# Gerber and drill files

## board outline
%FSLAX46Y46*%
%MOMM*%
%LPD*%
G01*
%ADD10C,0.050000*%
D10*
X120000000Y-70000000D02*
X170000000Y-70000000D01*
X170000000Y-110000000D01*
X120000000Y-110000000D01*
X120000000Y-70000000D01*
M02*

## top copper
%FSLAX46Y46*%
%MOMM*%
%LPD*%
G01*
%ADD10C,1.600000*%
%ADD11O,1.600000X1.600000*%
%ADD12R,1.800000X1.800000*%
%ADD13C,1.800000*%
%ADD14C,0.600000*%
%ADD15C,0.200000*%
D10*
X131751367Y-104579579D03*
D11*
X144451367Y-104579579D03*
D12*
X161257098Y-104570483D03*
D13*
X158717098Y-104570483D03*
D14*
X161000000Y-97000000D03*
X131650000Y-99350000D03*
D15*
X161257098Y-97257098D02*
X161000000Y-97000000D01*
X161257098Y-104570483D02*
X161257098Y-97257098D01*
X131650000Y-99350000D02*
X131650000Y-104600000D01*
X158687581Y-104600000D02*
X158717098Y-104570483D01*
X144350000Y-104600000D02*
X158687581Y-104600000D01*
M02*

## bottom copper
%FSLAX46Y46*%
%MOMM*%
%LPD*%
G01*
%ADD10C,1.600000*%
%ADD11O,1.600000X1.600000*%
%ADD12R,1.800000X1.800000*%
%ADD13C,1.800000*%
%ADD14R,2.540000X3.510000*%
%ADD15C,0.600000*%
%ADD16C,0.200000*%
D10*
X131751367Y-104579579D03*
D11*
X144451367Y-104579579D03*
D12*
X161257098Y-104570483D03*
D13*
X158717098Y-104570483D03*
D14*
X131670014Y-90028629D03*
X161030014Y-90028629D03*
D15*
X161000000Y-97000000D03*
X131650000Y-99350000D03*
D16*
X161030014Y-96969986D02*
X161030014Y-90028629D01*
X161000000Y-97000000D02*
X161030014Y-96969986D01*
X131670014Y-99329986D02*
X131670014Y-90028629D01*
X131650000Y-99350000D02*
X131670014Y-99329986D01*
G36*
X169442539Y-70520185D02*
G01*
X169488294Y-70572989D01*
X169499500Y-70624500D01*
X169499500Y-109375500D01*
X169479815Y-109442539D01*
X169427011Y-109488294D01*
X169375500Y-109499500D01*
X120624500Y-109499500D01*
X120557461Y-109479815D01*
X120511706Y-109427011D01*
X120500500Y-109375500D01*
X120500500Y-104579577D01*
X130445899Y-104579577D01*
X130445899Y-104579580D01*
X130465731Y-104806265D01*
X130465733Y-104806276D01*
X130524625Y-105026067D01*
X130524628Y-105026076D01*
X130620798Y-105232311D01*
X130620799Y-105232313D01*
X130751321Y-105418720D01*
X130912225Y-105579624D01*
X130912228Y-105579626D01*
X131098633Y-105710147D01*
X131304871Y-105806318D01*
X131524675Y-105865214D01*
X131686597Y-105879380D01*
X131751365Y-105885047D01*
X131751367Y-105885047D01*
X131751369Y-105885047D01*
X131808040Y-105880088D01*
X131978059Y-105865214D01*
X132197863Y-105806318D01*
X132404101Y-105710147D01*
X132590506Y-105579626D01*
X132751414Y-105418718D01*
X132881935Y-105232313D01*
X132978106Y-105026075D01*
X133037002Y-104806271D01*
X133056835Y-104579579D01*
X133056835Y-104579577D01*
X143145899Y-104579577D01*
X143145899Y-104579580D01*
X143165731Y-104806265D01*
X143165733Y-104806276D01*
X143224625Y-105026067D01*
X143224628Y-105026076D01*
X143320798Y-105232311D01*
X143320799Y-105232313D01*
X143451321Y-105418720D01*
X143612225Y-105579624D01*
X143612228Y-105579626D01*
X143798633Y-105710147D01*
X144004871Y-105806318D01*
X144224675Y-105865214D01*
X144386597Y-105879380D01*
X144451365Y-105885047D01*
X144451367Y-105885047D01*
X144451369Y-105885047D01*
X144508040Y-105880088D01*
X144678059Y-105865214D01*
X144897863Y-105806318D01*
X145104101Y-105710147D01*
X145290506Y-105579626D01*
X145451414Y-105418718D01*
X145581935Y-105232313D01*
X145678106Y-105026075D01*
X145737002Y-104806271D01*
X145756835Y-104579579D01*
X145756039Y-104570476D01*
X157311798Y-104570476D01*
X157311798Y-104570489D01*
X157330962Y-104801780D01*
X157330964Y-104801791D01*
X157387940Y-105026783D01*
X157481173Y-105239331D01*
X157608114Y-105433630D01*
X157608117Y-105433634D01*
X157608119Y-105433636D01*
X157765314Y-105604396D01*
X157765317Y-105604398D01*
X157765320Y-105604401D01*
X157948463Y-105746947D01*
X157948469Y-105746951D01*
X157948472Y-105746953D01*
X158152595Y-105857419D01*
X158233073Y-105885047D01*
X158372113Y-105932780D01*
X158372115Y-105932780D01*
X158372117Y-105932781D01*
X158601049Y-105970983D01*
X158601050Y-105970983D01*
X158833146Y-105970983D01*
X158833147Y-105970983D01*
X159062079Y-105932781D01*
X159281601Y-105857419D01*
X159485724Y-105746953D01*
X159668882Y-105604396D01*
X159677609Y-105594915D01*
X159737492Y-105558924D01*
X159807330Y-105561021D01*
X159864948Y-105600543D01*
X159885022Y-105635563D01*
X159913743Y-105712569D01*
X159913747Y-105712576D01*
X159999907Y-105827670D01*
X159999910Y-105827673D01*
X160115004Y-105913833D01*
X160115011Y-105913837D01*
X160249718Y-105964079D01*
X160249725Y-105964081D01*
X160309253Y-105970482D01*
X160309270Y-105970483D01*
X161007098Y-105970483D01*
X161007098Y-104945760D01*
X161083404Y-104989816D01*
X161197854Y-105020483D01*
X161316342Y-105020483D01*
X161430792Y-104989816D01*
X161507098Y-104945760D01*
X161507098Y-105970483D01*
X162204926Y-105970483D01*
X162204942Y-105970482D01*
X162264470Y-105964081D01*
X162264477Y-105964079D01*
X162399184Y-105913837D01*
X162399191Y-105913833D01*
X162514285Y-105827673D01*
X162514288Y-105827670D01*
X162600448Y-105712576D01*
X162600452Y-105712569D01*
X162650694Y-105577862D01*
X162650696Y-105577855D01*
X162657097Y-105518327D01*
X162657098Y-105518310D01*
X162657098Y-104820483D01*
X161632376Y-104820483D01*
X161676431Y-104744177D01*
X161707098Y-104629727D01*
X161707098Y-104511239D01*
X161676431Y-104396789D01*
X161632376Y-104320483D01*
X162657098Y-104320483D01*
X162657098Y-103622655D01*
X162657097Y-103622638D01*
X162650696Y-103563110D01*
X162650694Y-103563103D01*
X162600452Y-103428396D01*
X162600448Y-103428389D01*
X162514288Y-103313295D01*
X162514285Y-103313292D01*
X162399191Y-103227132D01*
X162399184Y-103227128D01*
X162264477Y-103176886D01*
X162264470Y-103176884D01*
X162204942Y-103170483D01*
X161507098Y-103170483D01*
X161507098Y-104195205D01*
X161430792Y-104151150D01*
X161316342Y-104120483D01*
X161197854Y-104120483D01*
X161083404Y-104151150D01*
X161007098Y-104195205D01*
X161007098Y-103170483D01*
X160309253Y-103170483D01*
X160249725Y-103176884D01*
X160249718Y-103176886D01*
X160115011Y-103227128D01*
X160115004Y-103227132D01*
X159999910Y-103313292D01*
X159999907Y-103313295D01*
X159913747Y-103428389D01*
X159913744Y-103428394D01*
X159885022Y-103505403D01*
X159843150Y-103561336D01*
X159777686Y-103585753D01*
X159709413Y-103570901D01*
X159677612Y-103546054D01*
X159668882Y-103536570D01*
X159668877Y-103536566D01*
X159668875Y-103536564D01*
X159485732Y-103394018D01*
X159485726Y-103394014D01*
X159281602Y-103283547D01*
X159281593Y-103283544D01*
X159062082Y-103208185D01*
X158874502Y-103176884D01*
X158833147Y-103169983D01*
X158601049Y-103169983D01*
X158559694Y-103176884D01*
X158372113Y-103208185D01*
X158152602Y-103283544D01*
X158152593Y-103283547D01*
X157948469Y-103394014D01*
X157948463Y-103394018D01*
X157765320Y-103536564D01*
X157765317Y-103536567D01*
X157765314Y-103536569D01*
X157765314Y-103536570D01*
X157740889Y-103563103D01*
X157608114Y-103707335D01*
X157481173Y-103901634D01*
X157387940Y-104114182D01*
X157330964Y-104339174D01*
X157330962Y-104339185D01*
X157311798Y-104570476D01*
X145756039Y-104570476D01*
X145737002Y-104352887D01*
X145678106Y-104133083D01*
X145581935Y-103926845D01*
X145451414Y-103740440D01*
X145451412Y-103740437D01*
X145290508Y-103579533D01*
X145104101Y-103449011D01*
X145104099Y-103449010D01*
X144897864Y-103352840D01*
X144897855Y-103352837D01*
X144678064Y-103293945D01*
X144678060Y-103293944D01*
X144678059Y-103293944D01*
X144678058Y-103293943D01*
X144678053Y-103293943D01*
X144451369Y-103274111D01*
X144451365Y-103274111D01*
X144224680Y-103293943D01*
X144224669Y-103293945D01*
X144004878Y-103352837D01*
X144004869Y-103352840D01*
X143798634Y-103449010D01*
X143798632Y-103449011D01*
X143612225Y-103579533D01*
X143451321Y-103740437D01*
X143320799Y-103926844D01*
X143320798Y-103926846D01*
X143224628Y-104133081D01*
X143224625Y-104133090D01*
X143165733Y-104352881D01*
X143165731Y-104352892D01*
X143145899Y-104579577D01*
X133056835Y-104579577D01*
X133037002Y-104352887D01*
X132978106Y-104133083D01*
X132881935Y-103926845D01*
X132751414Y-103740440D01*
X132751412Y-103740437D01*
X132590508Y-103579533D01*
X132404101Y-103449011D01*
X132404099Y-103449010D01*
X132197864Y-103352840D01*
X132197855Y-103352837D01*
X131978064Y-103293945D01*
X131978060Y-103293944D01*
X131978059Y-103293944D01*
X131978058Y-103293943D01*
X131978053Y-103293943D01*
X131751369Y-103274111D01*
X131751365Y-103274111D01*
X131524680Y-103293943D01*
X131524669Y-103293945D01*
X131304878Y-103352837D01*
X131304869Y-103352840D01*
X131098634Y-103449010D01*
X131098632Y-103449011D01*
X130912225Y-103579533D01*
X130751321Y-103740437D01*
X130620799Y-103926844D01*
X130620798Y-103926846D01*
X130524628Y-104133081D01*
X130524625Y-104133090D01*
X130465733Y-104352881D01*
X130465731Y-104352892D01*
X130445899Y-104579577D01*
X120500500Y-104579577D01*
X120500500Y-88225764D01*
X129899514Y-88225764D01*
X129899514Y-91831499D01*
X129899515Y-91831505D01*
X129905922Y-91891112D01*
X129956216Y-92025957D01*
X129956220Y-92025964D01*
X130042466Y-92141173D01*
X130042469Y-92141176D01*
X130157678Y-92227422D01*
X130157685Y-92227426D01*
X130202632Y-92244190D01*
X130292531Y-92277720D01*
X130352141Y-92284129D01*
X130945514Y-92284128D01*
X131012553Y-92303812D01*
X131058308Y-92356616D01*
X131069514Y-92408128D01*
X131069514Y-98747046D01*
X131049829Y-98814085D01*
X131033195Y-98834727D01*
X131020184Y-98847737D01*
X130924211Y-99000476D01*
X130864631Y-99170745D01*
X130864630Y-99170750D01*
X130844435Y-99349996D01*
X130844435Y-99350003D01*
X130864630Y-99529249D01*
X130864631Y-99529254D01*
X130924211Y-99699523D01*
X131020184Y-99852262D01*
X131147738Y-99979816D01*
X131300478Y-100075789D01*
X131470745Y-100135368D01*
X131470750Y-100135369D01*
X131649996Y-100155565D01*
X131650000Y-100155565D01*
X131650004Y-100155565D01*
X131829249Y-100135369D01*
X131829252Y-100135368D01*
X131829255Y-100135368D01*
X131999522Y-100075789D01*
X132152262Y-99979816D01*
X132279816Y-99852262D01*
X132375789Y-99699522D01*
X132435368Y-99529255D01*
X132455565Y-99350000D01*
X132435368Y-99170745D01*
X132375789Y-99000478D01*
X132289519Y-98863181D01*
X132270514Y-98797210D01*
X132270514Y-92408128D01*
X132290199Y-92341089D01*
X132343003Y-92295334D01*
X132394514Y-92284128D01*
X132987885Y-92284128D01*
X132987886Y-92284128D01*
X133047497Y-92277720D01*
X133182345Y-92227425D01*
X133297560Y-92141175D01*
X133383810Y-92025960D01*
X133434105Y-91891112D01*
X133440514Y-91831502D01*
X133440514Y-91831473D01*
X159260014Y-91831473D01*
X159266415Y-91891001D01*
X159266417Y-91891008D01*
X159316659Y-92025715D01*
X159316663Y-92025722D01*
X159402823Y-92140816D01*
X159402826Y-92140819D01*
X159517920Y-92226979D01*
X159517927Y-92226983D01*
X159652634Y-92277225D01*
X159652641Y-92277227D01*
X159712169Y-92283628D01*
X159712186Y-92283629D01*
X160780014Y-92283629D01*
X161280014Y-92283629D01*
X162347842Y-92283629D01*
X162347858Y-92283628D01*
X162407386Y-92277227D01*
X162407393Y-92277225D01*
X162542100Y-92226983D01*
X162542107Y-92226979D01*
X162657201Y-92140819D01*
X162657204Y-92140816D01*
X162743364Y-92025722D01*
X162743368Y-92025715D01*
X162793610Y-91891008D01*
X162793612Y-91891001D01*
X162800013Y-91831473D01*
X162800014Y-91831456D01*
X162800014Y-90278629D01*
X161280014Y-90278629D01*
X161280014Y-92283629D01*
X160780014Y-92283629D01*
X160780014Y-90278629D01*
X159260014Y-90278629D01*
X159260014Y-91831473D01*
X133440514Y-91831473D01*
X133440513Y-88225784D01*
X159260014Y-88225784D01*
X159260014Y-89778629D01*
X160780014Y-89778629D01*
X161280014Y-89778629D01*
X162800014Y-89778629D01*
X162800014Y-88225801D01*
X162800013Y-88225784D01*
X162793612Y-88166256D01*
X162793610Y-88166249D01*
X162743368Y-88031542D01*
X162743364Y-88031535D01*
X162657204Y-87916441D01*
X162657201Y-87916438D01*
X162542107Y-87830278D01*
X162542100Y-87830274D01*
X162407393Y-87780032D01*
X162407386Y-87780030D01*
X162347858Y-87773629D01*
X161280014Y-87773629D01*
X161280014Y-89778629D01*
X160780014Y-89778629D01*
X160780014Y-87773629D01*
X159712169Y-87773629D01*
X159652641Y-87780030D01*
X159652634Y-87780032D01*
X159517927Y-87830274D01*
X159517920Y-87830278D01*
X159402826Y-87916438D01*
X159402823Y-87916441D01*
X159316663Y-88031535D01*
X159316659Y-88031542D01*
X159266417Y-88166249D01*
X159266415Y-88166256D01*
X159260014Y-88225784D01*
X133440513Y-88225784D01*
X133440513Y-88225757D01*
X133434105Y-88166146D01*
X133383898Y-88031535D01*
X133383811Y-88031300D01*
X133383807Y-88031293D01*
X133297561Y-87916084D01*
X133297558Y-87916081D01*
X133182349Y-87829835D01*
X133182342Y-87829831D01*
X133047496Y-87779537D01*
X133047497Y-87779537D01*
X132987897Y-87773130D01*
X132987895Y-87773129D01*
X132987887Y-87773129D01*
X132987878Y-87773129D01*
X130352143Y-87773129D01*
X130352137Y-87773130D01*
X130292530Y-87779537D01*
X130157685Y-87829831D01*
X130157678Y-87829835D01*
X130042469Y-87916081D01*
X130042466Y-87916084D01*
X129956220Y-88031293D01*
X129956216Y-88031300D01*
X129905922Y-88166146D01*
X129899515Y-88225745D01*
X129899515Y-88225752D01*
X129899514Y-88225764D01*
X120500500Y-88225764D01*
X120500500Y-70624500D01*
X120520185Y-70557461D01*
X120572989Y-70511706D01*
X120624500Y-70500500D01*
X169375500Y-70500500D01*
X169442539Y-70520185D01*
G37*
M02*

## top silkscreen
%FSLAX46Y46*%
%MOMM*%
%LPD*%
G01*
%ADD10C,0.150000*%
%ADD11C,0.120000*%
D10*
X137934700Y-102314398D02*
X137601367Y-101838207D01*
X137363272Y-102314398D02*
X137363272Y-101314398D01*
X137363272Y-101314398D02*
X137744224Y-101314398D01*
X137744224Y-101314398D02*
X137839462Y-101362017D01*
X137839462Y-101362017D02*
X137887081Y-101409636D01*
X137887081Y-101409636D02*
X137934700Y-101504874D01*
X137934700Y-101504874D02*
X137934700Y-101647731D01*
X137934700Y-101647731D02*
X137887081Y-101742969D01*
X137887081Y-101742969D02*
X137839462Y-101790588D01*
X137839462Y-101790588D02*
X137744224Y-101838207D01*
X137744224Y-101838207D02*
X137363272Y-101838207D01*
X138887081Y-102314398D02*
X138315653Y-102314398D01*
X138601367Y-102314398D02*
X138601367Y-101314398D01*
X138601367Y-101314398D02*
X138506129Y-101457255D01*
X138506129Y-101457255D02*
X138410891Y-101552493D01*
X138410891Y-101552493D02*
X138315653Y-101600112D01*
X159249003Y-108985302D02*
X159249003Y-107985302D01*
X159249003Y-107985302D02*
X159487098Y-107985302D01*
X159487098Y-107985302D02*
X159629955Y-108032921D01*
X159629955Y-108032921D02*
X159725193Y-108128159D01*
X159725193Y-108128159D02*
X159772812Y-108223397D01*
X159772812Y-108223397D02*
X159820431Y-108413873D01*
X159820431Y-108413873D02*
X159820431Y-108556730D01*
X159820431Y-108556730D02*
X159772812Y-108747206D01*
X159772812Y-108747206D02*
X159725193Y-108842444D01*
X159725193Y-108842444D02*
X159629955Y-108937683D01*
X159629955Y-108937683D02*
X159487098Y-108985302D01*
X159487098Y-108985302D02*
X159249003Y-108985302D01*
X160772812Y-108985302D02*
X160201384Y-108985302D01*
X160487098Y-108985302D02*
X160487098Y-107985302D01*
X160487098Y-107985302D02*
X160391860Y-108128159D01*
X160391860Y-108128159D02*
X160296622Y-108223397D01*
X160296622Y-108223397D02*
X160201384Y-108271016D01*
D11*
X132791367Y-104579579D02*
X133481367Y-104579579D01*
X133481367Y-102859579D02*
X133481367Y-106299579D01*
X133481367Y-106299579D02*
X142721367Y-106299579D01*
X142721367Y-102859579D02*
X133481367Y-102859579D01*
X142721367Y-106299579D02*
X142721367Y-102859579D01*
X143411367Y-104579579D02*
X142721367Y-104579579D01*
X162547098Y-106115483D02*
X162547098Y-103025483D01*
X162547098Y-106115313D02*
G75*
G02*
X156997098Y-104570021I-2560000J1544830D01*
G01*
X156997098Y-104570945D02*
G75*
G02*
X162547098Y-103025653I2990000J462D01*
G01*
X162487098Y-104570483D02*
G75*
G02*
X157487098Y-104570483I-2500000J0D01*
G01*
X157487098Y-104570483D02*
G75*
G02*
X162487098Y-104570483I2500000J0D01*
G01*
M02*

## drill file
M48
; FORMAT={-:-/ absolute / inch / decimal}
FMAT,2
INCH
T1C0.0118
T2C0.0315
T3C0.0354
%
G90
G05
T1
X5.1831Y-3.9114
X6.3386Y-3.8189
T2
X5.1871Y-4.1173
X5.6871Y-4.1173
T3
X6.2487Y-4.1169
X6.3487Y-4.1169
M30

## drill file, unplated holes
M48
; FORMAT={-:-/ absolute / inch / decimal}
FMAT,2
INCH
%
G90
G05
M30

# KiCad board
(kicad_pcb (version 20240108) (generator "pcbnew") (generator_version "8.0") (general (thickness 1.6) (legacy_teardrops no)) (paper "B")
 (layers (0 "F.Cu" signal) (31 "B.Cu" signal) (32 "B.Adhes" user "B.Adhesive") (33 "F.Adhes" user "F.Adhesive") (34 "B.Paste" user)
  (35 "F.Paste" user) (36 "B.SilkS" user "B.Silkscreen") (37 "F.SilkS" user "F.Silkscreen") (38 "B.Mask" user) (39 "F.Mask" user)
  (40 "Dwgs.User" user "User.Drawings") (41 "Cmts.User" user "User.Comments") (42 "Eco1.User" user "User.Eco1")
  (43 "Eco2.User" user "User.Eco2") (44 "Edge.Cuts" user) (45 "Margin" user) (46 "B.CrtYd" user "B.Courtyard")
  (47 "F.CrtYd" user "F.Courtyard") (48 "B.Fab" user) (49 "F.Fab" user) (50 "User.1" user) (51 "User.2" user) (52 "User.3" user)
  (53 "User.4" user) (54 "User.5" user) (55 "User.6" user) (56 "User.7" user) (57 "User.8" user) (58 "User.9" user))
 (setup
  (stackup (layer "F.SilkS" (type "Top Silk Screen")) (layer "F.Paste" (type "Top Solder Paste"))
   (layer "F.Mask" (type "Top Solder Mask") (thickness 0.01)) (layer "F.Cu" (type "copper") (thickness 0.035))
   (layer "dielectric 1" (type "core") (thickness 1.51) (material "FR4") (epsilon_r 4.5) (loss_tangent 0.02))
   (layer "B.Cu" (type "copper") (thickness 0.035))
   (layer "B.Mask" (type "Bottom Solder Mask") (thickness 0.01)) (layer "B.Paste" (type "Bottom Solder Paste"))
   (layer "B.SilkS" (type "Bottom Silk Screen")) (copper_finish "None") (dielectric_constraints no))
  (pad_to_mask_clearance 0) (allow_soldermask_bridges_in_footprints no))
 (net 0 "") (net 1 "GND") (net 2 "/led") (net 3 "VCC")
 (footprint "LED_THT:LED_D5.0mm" (layer "F.Cu") (at 161.257098 104.570483 180)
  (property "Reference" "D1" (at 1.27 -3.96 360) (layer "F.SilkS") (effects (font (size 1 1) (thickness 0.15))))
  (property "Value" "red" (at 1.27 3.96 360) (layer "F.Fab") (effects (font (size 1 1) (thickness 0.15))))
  (fp_line (start -1.29 -1.545) (end -1.29 1.545) (stroke (width 0.12) (type solid)) (layer "F.SilkS"))
  (fp_arc (start 4.26 -0.000462) (mid 2.072002 2.880433) (end -1.29 1.54483) (stroke (width 0.12) (type solid)) (layer "F.SilkS"))
  (fp_arc (start -1.29 -1.54483) (mid 2.072002 -2.880433) (end 4.26 0.000462) (stroke (width 0.12) (type solid)) (layer "F.SilkS"))
  (fp_circle (center 1.27 0) (end 3.77 0) (stroke (width 0.12) (type solid)) (fill none) (layer "F.SilkS"))
  (pad "1" thru_hole rect (at 0 0 180) (size 1.8 1.8) (drill 0.9) (layers "*.Cu" "*.Mask") (remove_unused_layers no) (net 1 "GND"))
  (pad "2" thru_hole circle (at 2.54 0 180) (size 1.8 1.8) (drill 0.9) (layers "*.Cu" "*.Mask") (remove_unused_layers no) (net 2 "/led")))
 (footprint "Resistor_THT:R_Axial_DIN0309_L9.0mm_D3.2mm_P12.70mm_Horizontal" (layer "F.Cu") (at 131.751367 104.579579)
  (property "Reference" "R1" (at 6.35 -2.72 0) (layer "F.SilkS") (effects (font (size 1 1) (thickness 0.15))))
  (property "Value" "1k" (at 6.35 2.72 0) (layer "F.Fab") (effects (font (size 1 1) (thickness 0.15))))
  (fp_line (start 1.04 0) (end 1.73 0) (stroke (width 0.12) (type solid)) (layer "F.SilkS"))
  (fp_line (start 1.73 -1.72) (end 1.73 1.72) (stroke (width 0.12) (type solid)) (layer "F.SilkS"))
  (fp_line (start 1.73 1.72) (end 10.97 1.72) (stroke (width 0.12) (type solid)) (layer "F.SilkS"))
  (fp_line (start 10.97 -1.72) (end 1.73 -1.72) (stroke (width 0.12) (type solid)) (layer "F.SilkS"))
  (fp_line (start 10.97 1.72) (end 10.97 -1.72) (stroke (width 0.12) (type solid)) (layer "F.SilkS"))
  (fp_line (start 11.66 0) (end 10.97 0) (stroke (width 0.12) (type solid)) (layer "F.SilkS"))
  (pad "1" thru_hole circle (at 0 0) (size 1.6 1.6) (drill 0.8) (layers "*.Cu" "*.Mask") (remove_unused_layers no) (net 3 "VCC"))
  (pad "2" thru_hole oval (at 12.7 0) (size 1.6 1.6) (drill 0.8) (layers "*.Cu" "*.Mask") (remove_unused_layers no) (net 2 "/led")))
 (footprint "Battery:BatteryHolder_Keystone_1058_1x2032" (layer "B.Cu") (at 146.350014 90.028629)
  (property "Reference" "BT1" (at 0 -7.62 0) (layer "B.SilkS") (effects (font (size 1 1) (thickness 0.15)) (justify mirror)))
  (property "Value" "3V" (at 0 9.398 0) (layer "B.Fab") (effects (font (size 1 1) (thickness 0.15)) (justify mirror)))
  (pad "1" smd rect (at -14.68 0) (size 2.54 3.51) (layers "B.Cu" "B.Paste" "B.Mask") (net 3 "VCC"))
  (pad "2" smd rect (at 14.68 0) (size 2.54 3.51) (layers "B.Cu" "B.Paste" "B.Mask") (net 1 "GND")))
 (gr_rect (start 120 70) (end 170 110) (stroke (width 0.05) (type default)) (fill none) (layer "Edge.Cuts"))
 (segment (start 161.257098 104.570483) (end 161.257098 97.257098) (width 0.2) (layer "F.Cu") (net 1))
 (segment (start 161.257098 97.257098) (end 161 97) (width 0.2) (layer "F.Cu") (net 1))
 (via (at 161 97) (size 0.6) (drill 0.3) (layers "F.Cu" "B.Cu") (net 1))
 (segment (start 161 97) (end 161.030014 96.969986) (width 0.2) (layer "B.Cu") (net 1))
 (segment (start 161.030014 96.969986) (end 161.030014 90.028629) (width 0.2) (layer "B.Cu") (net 1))
 (segment (start 131.65 99.35) (end 131.65 104.6) (width 0.2) (layer "F.Cu") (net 3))
 (via (at 131.65 99.35) (size 0.6) (drill 0.3) (layers "F.Cu" "B.Cu") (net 3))
 (segment (start 131.65 99.35) (end 131.670014 99.329986) (width 0.2) (layer "B.Cu") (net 3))
 (segment (start 131.670014 99.329986) (end 131.670014 90.028629) (width 0.2) (layer "B.Cu") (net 3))
 (segment (start 144.35 104.6) (end 158.687581 104.6) (width 0.2) (layer "F.Cu") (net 2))
 (segment (start 158.687581 104.6) (end 158.717098 104.570483) (width 0.2) (layer "F.Cu") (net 2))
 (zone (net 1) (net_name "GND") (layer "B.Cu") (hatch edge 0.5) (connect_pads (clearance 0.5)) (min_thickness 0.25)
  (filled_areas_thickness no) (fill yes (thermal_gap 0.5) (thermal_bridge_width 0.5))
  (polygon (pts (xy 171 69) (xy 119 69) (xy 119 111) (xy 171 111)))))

